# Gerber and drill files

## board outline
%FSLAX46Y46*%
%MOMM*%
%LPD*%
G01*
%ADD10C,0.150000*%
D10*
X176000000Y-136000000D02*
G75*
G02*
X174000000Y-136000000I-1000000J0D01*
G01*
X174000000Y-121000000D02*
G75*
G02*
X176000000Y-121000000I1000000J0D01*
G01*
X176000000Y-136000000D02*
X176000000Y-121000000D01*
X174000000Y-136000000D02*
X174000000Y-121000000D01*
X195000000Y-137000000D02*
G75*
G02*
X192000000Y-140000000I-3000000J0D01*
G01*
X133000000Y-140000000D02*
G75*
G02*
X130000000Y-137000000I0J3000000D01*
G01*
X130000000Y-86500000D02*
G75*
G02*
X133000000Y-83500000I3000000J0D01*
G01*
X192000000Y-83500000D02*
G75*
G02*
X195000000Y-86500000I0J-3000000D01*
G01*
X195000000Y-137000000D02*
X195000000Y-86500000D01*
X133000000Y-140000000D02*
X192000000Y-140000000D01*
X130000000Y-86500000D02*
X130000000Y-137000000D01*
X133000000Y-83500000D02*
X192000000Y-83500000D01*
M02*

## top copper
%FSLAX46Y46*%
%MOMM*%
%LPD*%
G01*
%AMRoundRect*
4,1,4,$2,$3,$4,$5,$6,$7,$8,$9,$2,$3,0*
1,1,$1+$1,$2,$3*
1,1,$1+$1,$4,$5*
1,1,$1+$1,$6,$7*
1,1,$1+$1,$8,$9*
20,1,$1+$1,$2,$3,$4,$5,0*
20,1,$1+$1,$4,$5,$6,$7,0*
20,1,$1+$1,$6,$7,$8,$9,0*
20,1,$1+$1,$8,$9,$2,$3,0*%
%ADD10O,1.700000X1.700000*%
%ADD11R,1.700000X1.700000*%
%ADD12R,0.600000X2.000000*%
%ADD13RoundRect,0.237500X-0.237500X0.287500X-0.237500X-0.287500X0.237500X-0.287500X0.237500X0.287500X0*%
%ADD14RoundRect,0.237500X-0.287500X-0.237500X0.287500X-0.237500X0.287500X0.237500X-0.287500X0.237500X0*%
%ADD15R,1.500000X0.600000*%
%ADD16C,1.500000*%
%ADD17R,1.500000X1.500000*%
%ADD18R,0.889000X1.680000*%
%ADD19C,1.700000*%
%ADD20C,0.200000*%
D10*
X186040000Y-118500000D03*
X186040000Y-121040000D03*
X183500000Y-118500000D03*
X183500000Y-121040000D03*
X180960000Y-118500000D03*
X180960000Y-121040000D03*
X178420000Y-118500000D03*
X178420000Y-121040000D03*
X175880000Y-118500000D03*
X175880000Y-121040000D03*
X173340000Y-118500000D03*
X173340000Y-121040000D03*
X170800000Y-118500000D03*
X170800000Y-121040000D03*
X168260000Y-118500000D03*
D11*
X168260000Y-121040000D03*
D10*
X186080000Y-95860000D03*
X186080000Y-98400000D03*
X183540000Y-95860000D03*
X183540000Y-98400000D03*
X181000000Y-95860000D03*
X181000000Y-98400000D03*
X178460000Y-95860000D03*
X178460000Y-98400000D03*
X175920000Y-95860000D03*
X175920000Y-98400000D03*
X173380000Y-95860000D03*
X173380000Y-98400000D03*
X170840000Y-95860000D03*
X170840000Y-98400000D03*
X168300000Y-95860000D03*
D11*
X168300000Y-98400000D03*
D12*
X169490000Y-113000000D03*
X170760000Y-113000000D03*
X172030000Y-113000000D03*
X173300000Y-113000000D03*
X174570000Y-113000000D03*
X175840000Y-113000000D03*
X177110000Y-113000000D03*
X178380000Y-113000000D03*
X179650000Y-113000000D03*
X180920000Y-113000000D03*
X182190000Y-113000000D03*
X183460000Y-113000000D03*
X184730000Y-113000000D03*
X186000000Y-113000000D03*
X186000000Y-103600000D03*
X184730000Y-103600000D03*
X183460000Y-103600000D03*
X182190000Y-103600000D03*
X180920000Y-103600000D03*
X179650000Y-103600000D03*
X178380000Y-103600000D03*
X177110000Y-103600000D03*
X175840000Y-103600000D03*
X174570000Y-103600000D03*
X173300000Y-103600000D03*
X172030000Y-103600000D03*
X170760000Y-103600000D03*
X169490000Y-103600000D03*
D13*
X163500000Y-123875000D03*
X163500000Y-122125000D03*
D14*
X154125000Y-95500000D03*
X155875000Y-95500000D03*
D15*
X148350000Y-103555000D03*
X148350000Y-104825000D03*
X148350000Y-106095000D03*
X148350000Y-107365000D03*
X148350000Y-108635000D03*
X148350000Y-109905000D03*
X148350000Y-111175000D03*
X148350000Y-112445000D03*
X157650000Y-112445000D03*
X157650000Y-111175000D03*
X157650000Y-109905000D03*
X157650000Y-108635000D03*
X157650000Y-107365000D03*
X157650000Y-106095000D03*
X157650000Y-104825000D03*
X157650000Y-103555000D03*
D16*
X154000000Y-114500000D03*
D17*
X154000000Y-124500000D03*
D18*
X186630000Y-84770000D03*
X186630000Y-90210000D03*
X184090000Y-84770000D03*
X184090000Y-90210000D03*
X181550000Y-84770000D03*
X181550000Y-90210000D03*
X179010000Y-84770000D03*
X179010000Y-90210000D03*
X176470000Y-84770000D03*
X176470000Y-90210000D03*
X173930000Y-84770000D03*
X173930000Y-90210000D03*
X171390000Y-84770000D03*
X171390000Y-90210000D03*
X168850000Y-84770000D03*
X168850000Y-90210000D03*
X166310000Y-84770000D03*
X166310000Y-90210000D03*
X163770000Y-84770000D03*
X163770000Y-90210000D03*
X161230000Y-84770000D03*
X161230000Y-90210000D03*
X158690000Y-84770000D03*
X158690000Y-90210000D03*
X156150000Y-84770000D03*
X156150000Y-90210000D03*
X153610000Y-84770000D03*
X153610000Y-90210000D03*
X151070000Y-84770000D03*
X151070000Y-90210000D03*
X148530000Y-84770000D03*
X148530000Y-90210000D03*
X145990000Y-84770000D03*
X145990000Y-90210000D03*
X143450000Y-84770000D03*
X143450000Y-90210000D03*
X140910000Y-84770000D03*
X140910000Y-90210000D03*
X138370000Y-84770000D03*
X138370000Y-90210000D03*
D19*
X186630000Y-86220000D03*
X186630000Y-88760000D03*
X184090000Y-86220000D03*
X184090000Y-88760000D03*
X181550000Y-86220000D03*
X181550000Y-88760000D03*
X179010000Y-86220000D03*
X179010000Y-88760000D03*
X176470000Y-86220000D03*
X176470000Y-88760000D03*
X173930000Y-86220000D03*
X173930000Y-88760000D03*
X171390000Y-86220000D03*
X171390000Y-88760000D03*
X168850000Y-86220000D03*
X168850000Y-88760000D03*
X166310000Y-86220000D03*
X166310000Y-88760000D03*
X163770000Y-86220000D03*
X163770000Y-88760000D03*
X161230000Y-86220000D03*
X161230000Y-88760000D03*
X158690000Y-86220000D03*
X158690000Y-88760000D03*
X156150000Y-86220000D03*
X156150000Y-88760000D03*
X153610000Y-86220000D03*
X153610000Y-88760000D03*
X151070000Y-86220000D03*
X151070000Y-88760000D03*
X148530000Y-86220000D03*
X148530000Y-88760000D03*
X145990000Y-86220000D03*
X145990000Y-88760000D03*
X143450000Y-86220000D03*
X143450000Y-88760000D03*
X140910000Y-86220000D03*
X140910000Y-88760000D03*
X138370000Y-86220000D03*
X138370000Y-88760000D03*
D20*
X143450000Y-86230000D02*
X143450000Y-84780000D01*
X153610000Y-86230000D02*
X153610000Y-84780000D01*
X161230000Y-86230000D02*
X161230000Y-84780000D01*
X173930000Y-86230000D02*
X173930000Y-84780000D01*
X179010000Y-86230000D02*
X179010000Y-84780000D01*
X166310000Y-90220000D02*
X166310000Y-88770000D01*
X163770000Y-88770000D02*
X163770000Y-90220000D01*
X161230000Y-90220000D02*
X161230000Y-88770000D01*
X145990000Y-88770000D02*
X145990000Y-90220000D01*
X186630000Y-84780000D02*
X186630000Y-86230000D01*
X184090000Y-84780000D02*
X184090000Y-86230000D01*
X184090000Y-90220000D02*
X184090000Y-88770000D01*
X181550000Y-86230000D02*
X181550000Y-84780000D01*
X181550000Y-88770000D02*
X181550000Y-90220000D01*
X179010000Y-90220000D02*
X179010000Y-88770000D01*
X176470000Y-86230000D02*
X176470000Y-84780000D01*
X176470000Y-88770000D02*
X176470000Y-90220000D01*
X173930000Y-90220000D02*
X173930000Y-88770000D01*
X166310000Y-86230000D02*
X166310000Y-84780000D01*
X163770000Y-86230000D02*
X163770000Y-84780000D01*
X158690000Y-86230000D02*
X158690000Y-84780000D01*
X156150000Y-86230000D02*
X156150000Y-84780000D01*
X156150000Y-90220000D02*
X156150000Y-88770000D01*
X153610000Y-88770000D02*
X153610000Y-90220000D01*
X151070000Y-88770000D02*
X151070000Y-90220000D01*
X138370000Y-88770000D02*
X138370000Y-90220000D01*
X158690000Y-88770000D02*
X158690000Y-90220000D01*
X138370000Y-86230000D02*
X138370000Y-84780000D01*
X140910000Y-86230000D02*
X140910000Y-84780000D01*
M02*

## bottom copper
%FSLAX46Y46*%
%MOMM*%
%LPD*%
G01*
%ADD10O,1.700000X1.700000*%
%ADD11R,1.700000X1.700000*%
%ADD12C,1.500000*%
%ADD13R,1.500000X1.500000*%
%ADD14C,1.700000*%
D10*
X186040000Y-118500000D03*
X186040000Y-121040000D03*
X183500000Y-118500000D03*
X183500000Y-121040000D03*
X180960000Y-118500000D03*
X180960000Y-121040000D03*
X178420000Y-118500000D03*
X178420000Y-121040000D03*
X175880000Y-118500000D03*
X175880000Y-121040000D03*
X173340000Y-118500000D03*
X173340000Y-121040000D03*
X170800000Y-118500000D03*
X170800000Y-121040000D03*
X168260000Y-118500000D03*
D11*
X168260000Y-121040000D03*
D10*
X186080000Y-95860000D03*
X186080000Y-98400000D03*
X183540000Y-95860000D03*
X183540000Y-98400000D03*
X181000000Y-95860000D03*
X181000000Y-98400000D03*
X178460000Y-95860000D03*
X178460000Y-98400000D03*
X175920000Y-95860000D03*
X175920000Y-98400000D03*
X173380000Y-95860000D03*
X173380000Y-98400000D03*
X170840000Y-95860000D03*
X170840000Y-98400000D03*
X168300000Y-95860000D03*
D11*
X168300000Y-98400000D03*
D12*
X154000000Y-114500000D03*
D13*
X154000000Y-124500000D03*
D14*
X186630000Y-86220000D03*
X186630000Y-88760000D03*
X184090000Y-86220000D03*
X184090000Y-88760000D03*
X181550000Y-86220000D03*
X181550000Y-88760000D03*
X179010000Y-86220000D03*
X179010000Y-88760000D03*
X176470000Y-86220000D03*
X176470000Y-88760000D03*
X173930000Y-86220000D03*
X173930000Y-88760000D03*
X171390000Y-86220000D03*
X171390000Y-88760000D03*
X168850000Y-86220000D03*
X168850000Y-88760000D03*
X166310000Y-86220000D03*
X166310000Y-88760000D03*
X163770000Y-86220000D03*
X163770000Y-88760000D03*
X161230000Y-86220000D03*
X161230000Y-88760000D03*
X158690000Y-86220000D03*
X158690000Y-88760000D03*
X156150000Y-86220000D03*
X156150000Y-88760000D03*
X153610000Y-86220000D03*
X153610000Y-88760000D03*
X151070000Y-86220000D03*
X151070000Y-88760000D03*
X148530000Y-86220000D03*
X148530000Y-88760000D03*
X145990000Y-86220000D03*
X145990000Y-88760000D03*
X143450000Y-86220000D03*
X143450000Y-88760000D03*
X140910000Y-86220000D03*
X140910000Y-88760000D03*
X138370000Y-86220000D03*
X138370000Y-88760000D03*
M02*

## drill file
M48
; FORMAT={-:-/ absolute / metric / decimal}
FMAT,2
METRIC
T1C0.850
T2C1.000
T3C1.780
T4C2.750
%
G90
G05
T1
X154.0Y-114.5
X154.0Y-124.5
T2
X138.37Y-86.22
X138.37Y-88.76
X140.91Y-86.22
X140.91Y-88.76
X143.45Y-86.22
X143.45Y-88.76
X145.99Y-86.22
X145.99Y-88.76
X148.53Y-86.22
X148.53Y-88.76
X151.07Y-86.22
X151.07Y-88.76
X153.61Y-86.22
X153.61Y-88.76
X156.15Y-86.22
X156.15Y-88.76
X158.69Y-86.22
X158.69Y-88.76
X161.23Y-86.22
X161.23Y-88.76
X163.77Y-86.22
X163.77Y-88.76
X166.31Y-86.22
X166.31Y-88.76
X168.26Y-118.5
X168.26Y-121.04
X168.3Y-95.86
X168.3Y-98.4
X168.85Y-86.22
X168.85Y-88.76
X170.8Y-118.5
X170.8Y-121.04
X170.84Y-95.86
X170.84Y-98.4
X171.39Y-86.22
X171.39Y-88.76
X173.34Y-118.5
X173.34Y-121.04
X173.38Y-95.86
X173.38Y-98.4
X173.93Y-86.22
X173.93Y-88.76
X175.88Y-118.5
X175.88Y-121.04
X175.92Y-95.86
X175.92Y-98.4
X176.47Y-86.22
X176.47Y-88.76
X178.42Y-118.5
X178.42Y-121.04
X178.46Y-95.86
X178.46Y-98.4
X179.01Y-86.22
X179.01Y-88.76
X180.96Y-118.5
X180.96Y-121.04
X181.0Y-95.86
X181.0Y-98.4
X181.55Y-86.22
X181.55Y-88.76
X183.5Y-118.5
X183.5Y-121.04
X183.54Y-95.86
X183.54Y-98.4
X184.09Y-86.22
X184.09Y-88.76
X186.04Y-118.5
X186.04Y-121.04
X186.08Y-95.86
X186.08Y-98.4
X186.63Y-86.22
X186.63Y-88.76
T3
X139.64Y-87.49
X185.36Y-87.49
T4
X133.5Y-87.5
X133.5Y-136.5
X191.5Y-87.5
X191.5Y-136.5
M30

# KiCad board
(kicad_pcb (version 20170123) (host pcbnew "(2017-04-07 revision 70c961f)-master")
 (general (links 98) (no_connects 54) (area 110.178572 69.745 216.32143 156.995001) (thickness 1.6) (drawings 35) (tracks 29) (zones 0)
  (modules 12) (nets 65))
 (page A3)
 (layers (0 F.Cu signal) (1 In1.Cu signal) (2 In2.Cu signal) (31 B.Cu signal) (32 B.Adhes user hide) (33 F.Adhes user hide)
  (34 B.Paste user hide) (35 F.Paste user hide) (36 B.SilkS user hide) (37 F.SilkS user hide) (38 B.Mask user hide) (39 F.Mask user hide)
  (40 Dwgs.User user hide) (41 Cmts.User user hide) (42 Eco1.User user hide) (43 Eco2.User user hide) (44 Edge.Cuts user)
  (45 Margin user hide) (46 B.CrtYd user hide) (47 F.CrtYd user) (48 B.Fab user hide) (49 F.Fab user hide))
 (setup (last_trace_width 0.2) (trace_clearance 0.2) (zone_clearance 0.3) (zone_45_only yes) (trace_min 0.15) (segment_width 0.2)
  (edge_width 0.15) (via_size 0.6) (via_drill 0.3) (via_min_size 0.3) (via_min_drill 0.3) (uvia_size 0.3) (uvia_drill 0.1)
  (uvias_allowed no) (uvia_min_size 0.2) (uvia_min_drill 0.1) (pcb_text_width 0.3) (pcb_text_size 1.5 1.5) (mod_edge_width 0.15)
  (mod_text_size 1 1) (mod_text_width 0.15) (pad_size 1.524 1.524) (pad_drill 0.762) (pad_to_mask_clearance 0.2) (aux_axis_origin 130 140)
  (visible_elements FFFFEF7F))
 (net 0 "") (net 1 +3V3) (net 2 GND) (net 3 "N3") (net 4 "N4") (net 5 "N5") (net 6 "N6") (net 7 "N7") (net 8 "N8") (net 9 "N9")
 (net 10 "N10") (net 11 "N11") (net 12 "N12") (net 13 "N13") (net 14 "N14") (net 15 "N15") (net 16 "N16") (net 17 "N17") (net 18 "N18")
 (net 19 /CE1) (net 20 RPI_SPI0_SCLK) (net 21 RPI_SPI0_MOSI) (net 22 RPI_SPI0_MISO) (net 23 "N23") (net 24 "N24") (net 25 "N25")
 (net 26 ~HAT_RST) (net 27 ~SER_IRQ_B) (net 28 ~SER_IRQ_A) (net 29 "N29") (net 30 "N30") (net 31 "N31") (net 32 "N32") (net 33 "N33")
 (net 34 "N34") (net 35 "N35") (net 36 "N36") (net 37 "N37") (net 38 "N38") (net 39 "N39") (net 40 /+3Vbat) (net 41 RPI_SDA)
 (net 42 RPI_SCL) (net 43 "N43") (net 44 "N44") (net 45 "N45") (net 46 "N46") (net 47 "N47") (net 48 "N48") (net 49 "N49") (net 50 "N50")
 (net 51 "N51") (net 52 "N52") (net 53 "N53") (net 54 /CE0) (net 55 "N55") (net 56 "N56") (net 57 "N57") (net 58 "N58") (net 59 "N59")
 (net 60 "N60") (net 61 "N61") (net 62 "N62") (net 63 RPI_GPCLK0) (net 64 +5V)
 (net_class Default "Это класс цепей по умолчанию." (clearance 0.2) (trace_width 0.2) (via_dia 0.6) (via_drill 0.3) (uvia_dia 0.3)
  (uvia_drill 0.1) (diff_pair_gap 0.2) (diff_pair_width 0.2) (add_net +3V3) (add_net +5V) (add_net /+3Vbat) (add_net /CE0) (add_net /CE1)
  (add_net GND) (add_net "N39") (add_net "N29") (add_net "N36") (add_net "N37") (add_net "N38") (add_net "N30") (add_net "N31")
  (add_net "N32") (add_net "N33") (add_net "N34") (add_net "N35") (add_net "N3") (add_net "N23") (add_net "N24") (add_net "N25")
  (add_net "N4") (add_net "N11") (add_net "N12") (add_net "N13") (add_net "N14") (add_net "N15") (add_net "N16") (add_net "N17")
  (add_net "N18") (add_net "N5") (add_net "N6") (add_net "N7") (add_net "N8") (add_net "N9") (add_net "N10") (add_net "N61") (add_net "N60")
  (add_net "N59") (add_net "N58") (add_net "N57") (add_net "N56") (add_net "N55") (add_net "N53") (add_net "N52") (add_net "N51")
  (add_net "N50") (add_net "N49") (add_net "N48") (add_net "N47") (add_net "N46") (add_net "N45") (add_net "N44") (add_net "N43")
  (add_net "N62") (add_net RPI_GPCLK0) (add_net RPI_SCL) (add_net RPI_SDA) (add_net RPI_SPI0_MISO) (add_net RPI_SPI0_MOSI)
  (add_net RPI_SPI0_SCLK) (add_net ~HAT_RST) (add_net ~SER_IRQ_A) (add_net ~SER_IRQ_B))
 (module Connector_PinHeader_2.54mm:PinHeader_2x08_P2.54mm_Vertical (layer F.Cu) (at 168.26 121.04 90)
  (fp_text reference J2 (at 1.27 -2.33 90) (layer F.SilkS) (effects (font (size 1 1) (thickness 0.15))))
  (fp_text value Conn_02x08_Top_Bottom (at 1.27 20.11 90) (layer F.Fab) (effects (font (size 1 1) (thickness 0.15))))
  (pad 16 thru_hole oval (at 2.54 17.78 90) (size 1.7 1.7) (drill 1) (layers *.Cu *.Mask) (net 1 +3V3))
  (pad 15 thru_hole oval (at 0 17.78 90) (size 1.7 1.7) (drill 1) (layers *.Cu *.Mask) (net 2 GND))
  (pad 14 thru_hole oval (at 2.54 15.24 90) (size 1.7 1.7) (drill 1) (layers *.Cu *.Mask) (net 1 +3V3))
  (pad 13 thru_hole oval (at 0 15.24 90) (size 1.7 1.7) (drill 1) (layers *.Cu *.Mask) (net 2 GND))
  (pad 12 thru_hole oval (at 2.54 12.7 90) (size 1.7 1.7) (drill 1) (layers *.Cu *.Mask) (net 1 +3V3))
  (pad 11 thru_hole oval (at 0 12.7 90) (size 1.7 1.7) (drill 1) (layers *.Cu *.Mask) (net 2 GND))
  (pad 10 thru_hole oval (at 2.54 10.16 90) (size 1.7 1.7) (drill 1) (layers *.Cu *.Mask) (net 1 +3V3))
  (pad 9 thru_hole oval (at 0 10.16 90) (size 1.7 1.7) (drill 1) (layers *.Cu *.Mask) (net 2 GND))
  (pad 8 thru_hole oval (at 2.54 7.62 90) (size 1.7 1.7) (drill 1) (layers *.Cu *.Mask) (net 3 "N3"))
  (pad 7 thru_hole oval (at 0 7.62 90) (size 1.7 1.7) (drill 1) (layers *.Cu *.Mask) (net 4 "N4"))
  (pad 6 thru_hole oval (at 2.54 5.08 90) (size 1.7 1.7) (drill 1) (layers *.Cu *.Mask) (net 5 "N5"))
  (pad 5 thru_hole oval (at 0 5.08 90) (size 1.7 1.7) (drill 1) (layers *.Cu *.Mask) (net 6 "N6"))
  (pad 4 thru_hole oval (at 2.54 2.54 90) (size 1.7 1.7) (drill 1) (layers *.Cu *.Mask) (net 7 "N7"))
  (pad 3 thru_hole oval (at 0 2.54 90) (size 1.7 1.7) (drill 1) (layers *.Cu *.Mask) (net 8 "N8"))
  (pad 2 thru_hole oval (at 2.54 0 90) (size 1.7 1.7) (drill 1) (layers *.Cu *.Mask) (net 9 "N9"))
  (pad 1 thru_hole rect (at 0 0 90) (size 1.7 1.7) (drill 1) (layers *.Cu *.Mask) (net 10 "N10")))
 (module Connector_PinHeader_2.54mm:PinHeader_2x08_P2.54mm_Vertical (layer F.Cu) (at 168.3 98.4 90)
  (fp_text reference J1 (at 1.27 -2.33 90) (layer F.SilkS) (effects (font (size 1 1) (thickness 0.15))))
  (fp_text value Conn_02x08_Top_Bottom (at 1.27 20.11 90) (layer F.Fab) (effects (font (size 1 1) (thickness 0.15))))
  (pad 16 thru_hole oval (at 2.54 17.78 90) (size 1.7 1.7) (drill 1) (layers *.Cu *.Mask) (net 1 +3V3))
  (pad 15 thru_hole oval (at 0 17.78 90) (size 1.7 1.7) (drill 1) (layers *.Cu *.Mask) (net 2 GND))
  (pad 14 thru_hole oval (at 2.54 15.24 90) (size 1.7 1.7) (drill 1) (layers *.Cu *.Mask) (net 1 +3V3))
  (pad 13 thru_hole oval (at 0 15.24 90) (size 1.7 1.7) (drill 1) (layers *.Cu *.Mask) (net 2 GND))
  (pad 12 thru_hole oval (at 2.54 12.7 90) (size 1.7 1.7) (drill 1) (layers *.Cu *.Mask) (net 1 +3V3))
  (pad 11 thru_hole oval (at 0 12.7 90) (size 1.7 1.7) (drill 1) (layers *.Cu *.Mask) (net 2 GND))
  (pad 10 thru_hole oval (at 2.54 10.16 90) (size 1.7 1.7) (drill 1) (layers *.Cu *.Mask) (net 1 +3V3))
  (pad 9 thru_hole oval (at 0 10.16 90) (size 1.7 1.7) (drill 1) (layers *.Cu *.Mask) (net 2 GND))
  (pad 8 thru_hole oval (at 2.54 7.62 90) (size 1.7 1.7) (drill 1) (layers *.Cu *.Mask) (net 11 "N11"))
  (pad 7 thru_hole oval (at 0 7.62 90) (size 1.7 1.7) (drill 1) (layers *.Cu *.Mask) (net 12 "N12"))
  (pad 6 thru_hole oval (at 2.54 5.08 90) (size 1.7 1.7) (drill 1) (layers *.Cu *.Mask) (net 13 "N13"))
  (pad 5 thru_hole oval (at 0 5.08 90) (size 1.7 1.7) (drill 1) (layers *.Cu *.Mask) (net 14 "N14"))
  (pad 4 thru_hole oval (at 2.54 2.54 90) (size 1.7 1.7) (drill 1) (layers *.Cu *.Mask) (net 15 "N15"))
  (pad 3 thru_hole oval (at 0 2.54 90) (size 1.7 1.7) (drill 1) (layers *.Cu *.Mask) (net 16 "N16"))
  (pad 2 thru_hole oval (at 2.54 0 90) (size 1.7 1.7) (drill 1) (layers *.Cu *.Mask) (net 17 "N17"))
  (pad 1 thru_hole rect (at 0 0 90) (size 1.7 1.7) (drill 1) (layers *.Cu *.Mask) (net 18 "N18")))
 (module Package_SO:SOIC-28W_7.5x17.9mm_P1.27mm (layer F.Cu) (at 177.745 108.3 90)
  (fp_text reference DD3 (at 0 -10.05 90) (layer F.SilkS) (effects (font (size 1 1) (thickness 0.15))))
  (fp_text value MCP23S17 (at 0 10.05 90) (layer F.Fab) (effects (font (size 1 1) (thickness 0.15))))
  (pad 1 smd rect (at -4.7 -8.255 90) (size 2 0.6) (layers F.Cu F.Paste F.Mask) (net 3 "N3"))
  (pad 2 smd rect (at -4.7 -6.985 90) (size 2 0.6) (layers F.Cu F.Paste F.Mask) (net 4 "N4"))
  (pad 3 smd rect (at -4.7 -5.715 90) (size 2 0.6) (layers F.Cu F.Paste F.Mask) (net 5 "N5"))
  (pad 4 smd rect (at -4.7 -4.445 90) (size 2 0.6) (layers F.Cu F.Paste F.Mask) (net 6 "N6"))
  (pad 5 smd rect (at -4.7 -3.175 90) (size 2 0.6) (layers F.Cu F.Paste F.Mask) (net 7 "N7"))
  (pad 6 smd rect (at -4.7 -1.905 90) (size 2 0.6) (layers F.Cu F.Paste F.Mask) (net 8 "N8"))
  (pad 7 smd rect (at -4.7 -0.635 90) (size 2 0.6) (layers F.Cu F.Paste F.Mask) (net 9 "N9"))
  (pad 8 smd rect (at -4.7 0.635 90) (size 2 0.6) (layers F.Cu F.Paste F.Mask) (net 10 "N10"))
  (pad 9 smd rect (at -4.7 1.905 90) (size 2 0.6) (layers F.Cu F.Paste F.Mask) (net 1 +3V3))
  (pad 10 smd rect (at -4.7 3.175 90) (size 2 0.6) (layers F.Cu F.Paste F.Mask) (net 2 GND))
  (pad 11 smd rect (at -4.7 4.445 90) (size 2 0.6) (layers F.Cu F.Paste F.Mask) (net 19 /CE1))
  (pad 12 smd rect (at -4.7 5.715 90) (size 2 0.6) (layers F.Cu F.Paste F.Mask) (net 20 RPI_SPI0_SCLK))
  (pad 13 smd rect (at -4.7 6.985 90) (size 2 0.6) (layers F.Cu F.Paste F.Mask) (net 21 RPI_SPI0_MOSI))
  (pad 14 smd rect (at -4.7 8.255 90) (size 2 0.6) (layers F.Cu F.Paste F.Mask) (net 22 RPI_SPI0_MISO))
  (pad 15 smd rect (at 4.7 8.255 90) (size 2 0.6) (layers F.Cu F.Paste F.Mask) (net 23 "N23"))
  (pad 16 smd rect (at 4.7 6.985 90) (size 2 0.6) (layers F.Cu F.Paste F.Mask) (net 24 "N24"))
  (pad 17 smd rect (at 4.7 5.715 90) (size 2 0.6) (layers F.Cu F.Paste F.Mask) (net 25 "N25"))
  (pad 18 smd rect (at 4.7 4.445 90) (size 2 0.6) (layers F.Cu F.Paste F.Mask) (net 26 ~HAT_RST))
  (pad 19 smd rect (at 4.7 3.175 90) (size 2 0.6) (layers F.Cu F.Paste F.Mask) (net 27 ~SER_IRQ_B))
  (pad 20 smd rect (at 4.7 1.905 90) (size 2 0.6) (layers F.Cu F.Paste F.Mask) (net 27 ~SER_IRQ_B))
  (pad 21 smd rect (at 4.7 0.635 90) (size 2 0.6) (layers F.Cu F.Paste F.Mask) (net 11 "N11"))
  (pad 22 smd rect (at 4.7 -0.635 90) (size 2 0.6) (layers F.Cu F.Paste F.Mask) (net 12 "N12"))
  (pad 23 smd rect (at 4.7 -1.905 90) (size 2 0.6) (layers F.Cu F.Paste F.Mask) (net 13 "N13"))
  (pad 24 smd rect (at 4.7 -3.175 90) (size 2 0.6) (layers F.Cu F.Paste F.Mask) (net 14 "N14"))
  (pad 25 smd rect (at 4.7 -4.445 90) (size 2 0.6) (layers F.Cu F.Paste F.Mask) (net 15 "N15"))
  (pad 26 smd rect (at 4.7 -5.715 90) (size 2 0.6) (layers F.Cu F.Paste F.Mask) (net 16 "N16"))
  (pad 27 smd rect (at 4.7 -6.985 90) (size 2 0.6) (layers F.Cu F.Paste F.Mask) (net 17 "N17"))
  (pad 28 smd rect (at 4.7 -8.255 90) (size 2 0.6) (layers F.Cu F.Paste F.Mask) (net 18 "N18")))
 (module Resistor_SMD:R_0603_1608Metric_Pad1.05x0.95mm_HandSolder (layer F.Cu) (at 163.5 123 270)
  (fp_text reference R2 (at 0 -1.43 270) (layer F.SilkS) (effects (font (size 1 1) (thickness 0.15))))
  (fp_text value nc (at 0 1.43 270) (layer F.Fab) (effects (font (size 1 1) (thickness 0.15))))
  (pad 2 smd roundrect (at 0.875 0 270) (size 1.05 0.95) (layers F.Cu F.Paste F.Mask) (roundrect_rratio 0.25) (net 1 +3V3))
  (pad 1 smd roundrect (at -0.875 0 270) (size 1.05 0.95) (layers F.Cu F.Paste F.Mask) (roundrect_rratio 0.25) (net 26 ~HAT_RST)))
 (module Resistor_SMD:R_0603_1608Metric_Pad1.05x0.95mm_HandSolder (layer F.Cu) (at 155 95.5)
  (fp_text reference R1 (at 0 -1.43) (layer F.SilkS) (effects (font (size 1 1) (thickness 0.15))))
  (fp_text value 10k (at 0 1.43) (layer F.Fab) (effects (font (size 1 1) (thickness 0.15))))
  (pad 1 smd roundrect (at -0.875 0) (size 1.05 0.95) (layers F.Cu F.Paste F.Mask) (roundrect_rratio 0.25) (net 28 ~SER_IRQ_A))
  (pad 2 smd roundrect (at 0.875 0) (size 1.05 0.95) (layers F.Cu F.Paste F.Mask) (roundrect_rratio 0.25) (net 1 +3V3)))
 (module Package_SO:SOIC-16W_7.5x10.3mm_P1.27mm (layer F.Cu) (at 153 108)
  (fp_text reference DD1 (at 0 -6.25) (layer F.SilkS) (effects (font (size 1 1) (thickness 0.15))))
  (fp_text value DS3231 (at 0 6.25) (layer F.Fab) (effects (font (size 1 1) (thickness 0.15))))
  (pad 1 smd rect (at -4.65 -4.445) (size 1.5 0.6) (layers F.Cu F.Paste F.Mask) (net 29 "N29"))
  (pad 2 smd rect (at -4.65 -3.175) (size 1.5 0.6) (layers F.Cu F.Paste F.Mask) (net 1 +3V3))
  (pad 3 smd rect (at -4.65 -1.905) (size 1.5 0.6) (layers F.Cu F.Paste F.Mask) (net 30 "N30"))
  (pad 4 smd rect (at -4.65 -0.635) (size 1.5 0.6) (layers F.Cu F.Paste F.Mask) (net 26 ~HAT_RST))
  (pad 5 smd rect (at -4.65 0.635) (size 1.5 0.6) (layers F.Cu F.Paste F.Mask) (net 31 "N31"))
  (pad 6 smd rect (at -4.65 1.905) (size 1.5 0.6) (layers F.Cu F.Paste F.Mask) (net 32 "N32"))
  (pad 7 smd rect (at -4.65 3.175) (size 1.5 0.6) (layers F.Cu F.Paste F.Mask) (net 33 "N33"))
  (pad 8 smd rect (at -4.65 4.445) (size 1.5 0.6) (layers F.Cu F.Paste F.Mask) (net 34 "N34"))
  (pad 9 smd rect (at 4.65 4.445) (size 1.5 0.6) (layers F.Cu F.Paste F.Mask) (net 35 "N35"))
  (pad 10 smd rect (at 4.65 3.175) (size 1.5 0.6) (layers F.Cu F.Paste F.Mask) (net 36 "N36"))
  (pad 11 smd rect (at 4.65 1.905) (size 1.5 0.6) (layers F.Cu F.Paste F.Mask) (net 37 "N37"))
  (pad 12 smd rect (at 4.65 0.635) (size 1.5 0.6) (layers F.Cu F.Paste F.Mask) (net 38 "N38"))
  (pad 13 smd rect (at 4.65 -0.635) (size 1.5 0.6) (layers F.Cu F.Paste F.Mask) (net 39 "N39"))
  (pad 14 smd rect (at 4.65 -1.905) (size 1.5 0.6) (layers F.Cu F.Paste F.Mask) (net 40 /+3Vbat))
  (pad 15 smd rect (at 4.65 -3.175) (size 1.5 0.6) (layers F.Cu F.Paste F.Mask) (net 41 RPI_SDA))
  (pad 16 smd rect (at 4.65 -4.445) (size 1.5 0.6) (layers F.Cu F.Paste F.Mask) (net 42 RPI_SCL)))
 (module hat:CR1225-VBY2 (layer F.Cu) (at 154 119.5 90)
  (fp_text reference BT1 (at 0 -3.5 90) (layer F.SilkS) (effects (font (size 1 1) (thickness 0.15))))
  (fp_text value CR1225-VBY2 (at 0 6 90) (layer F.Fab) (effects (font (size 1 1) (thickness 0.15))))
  (pad 2 thru_hole circle (at 5 0 90) (size 1.5 1.5) (drill 0.85) (layers *.Cu *.Mask) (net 39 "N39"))
  (pad 1 thru_hole rect (at -5 0 90) (size 1.5 1.5) (drill 0.85) (layers *.Cu *.Mask) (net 40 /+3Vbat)))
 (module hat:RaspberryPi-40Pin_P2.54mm (layer F.Cu) (at 162.5 87.49)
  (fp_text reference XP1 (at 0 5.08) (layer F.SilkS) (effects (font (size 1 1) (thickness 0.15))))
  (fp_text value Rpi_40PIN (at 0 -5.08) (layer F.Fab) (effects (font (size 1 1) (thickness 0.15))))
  (pad "" np_thru_hole circle (at 22.86 0) (size 1.78 1.78) (drill 1.78) (layers *.Cu *.Mask))
  (pad "" np_thru_hole circle (at -22.86 0) (size 1.78 1.78) (drill 1.78) (layers *.Cu *.Mask))
  (pad 40 smd rect (at 24.13 -2.72) (size 0.889 1.68) (layers F.Cu F.Paste F.Mask) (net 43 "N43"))
  (pad 39 smd rect (at 24.13 2.72) (size 0.889 1.68) (layers F.Cu F.Paste F.Mask) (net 2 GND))
  (pad 38 smd rect (at 21.59 -2.72) (size 0.889 1.68) (layers F.Cu F.Paste F.Mask) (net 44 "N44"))
  (pad 37 smd rect (at 21.59 2.72) (size 0.889 1.68) (layers F.Cu F.Paste F.Mask) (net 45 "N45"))
  (pad 36 smd rect (at 19.05 -2.72) (size 0.889 1.68) (layers F.Cu F.Paste F.Mask) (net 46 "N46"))
  (pad 35 smd rect (at 19.05 2.72) (size 0.889 1.68) (layers F.Cu F.Paste F.Mask) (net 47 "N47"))
  (pad 34 smd rect (at 16.51 -2.72) (size 0.889 1.68) (layers F.Cu F.Paste F.Mask) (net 2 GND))
  (pad 33 smd rect (at 16.51 2.72) (size 0.889 1.68) (layers F.Cu F.Paste F.Mask) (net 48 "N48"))
  (pad 32 smd rect (at 13.97 -2.72) (size 0.889 1.68) (layers F.Cu F.Paste F.Mask) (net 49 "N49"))
  (pad 31 smd rect (at 13.97 2.72) (size 0.889 1.68) (layers F.Cu F.Paste F.Mask) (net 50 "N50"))
  (pad 30 smd rect (at 11.43 -2.72) (size 0.889 1.68) (layers F.Cu F.Paste F.Mask) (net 2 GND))
  (pad 29 smd rect (at 11.43 2.72) (size 0.889 1.68) (layers F.Cu F.Paste F.Mask) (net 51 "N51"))
  (pad 28 smd rect (at 8.89 -2.72) (size 0.889 1.68) (layers F.Cu F.Paste F.Mask) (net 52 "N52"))
  (pad 27 smd rect (at 8.89 2.72) (size 0.889 1.68) (layers F.Cu F.Paste F.Mask) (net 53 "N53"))
  (pad 26 smd rect (at 6.35 -2.72) (size 0.889 1.68) (layers F.Cu F.Paste F.Mask) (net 19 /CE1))
  (pad 25 smd rect (at 6.35 2.72) (size 0.889 1.68) (layers F.Cu F.Paste F.Mask) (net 2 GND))
  (pad 24 smd rect (at 3.81 -2.72) (size 0.889 1.68) (layers F.Cu F.Paste F.Mask) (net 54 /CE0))
  (pad 23 smd rect (at 3.81 2.72) (size 0.889 1.68) (layers F.Cu F.Paste F.Mask) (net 20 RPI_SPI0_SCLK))
  (pad 22 smd rect (at 1.27 -2.72) (size 0.889 1.68) (layers F.Cu F.Paste F.Mask) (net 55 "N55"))
  (pad 21 smd rect (at 1.27 2.72) (size 0.889 1.68) (layers F.Cu F.Paste F.Mask) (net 22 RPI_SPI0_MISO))
  (pad 20 smd rect (at -1.27 -2.72) (size 0.889 1.68) (layers F.Cu F.Paste F.Mask) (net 2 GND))
  (pad 19 smd rect (at -1.27 2.72) (size 0.889 1.68) (layers F.Cu F.Paste F.Mask) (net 21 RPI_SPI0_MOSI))
  (pad 18 smd rect (at -3.81 -2.72) (size 0.889 1.68) (layers F.Cu F.Paste F.Mask) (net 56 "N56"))
  (pad 17 smd rect (at -3.81 2.72) (size 0.889 1.68) (layers F.Cu F.Paste F.Mask) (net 1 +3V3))
  (pad 16 smd rect (at -6.35 -2.72) (size 0.889 1.68) (layers F.Cu F.Paste F.Mask) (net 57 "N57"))
  (pad 15 smd rect (at -6.35 2.72) (size 0.889 1.68) (layers F.Cu F.Paste F.Mask) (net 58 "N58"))
  (pad 14 smd rect (at -8.89 -2.72) (size 0.889 1.68) (layers F.Cu F.Paste F.Mask) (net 2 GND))
  (pad 13 smd rect (at -8.89 2.72) (size 0.889 1.68) (layers F.Cu F.Paste F.Mask) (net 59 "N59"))
  (pad 12 smd rect (at -11.43 -2.72) (size 0.889 1.68) (layers F.Cu F.Paste F.Mask) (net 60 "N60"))
  (pad 11 smd rect (at -11.43 2.72) (size 0.889 1.68) (layers F.Cu F.Paste F.Mask) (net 28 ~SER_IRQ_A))
  (pad 10 smd rect (at -13.97 -2.72) (size 0.889 1.68) (layers F.Cu F.Paste F.Mask) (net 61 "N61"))
  (pad 9 smd rect (at -13.97 2.72) (size 0.889 1.68) (layers F.Cu F.Paste F.Mask) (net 2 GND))
  (pad 8 smd rect (at -16.51 -2.72) (size 0.889 1.68) (layers F.Cu F.Paste F.Mask) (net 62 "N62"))
  (pad 7 smd rect (at -16.51 2.72) (size 0.889 1.68) (layers F.Cu F.Paste F.Mask) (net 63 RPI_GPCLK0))
  (pad 6 smd rect (at -19.05 -2.72) (size 0.889 1.68) (layers F.Cu F.Paste F.Mask) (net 2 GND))
  (pad 5 smd rect (at -19.05 2.72) (size 0.889 1.68) (layers F.Cu F.Paste F.Mask) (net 42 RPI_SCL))
  (pad 4 smd rect (at -21.59 -2.72) (size 0.889 1.68) (layers F.Cu F.Paste F.Mask) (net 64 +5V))
  (pad 3 smd rect (at -21.59 2.72) (size 0.889 1.68) (layers F.Cu F.Paste F.Mask) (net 41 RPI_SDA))
  (pad 2 smd rect (at -24.13 -2.72) (size 0.889 1.68) (layers F.Cu F.Paste F.Mask) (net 64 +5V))
  (pad 1 smd rect (at -24.13 2.72) (size 0.889 1.68) (layers F.Cu F.Paste F.Mask) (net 1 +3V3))
  (pad 40 thru_hole circle (at 24.13 -1.27) (size 1.7 1.7) (drill 1) (layers *.Cu *.Mask) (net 43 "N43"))
  (pad 39 thru_hole circle (at 24.13 1.27) (size 1.7 1.7) (drill 1) (layers *.Cu *.Mask) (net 2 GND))
  (pad 38 thru_hole circle (at 21.59 -1.27) (size 1.7 1.7) (drill 1) (layers *.Cu *.Mask) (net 44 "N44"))
  (pad 37 thru_hole circle (at 21.59 1.27) (size 1.7 1.7) (drill 1) (layers *.Cu *.Mask) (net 45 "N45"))
  (pad 36 thru_hole circle (at 19.05 -1.27) (size 1.7 1.7) (drill 1) (layers *.Cu *.Mask) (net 46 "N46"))
  (pad 35 thru_hole circle (at 19.05 1.27) (size 1.7 1.7) (drill 1) (layers *.Cu *.Mask) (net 47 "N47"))
  (pad 34 thru_hole circle (at 16.51 -1.27) (size 1.7 1.7) (drill 1) (layers *.Cu *.Mask) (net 2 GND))
  (pad 33 thru_hole circle (at 16.51 1.27) (size 1.7 1.7) (drill 1) (layers *.Cu *.Mask) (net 48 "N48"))
  (pad 32 thru_hole circle (at 13.97 -1.27) (size 1.7 1.7) (drill 1) (layers *.Cu *.Mask) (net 49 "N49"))
  (pad 31 thru_hole circle (at 13.97 1.27) (size 1.7 1.7) (drill 1) (layers *.Cu *.Mask) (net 50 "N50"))
  (pad 30 thru_hole circle (at 11.43 -1.27) (size 1.7 1.7) (drill 1) (layers *.Cu *.Mask) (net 2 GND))
  (pad 29 thru_hole circle (at 11.43 1.27) (size 1.7 1.7) (drill 1) (layers *.Cu *.Mask) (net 51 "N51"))
  (pad 28 thru_hole circle (at 8.89 -1.27) (size 1.7 1.7) (drill 1) (layers *.Cu *.Mask) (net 52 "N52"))
  (pad 27 thru_hole circle (at 8.89 1.27) (size 1.7 1.7) (drill 1) (layers *.Cu *.Mask) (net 53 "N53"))
  (pad 26 thru_hole circle (at 6.35 -1.27) (size 1.7 1.7) (drill 1) (layers *.Cu *.Mask) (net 19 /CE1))
  (pad 25 thru_hole circle (at 6.35 1.27) (size 1.7 1.7) (drill 1) (layers *.Cu *.Mask) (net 2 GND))
  (pad 24 thru_hole circle (at 3.81 -1.27) (size 1.7 1.7) (drill 1) (layers *.Cu *.Mask) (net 54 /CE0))
  (pad 23 thru_hole circle (at 3.81 1.27) (size 1.7 1.7) (drill 1) (layers *.Cu *.Mask) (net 20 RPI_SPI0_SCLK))
  (pad 22 thru_hole circle (at 1.27 -1.27) (size 1.7 1.7) (drill 1) (layers *.Cu *.Mask) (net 55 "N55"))
  (pad 21 thru_hole circle (at 1.27 1.27) (size 1.7 1.7) (drill 1) (layers *.Cu *.Mask) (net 22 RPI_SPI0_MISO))
  (pad 20 thru_hole circle (at -1.27 -1.27) (size 1.7 1.7) (drill 1) (layers *.Cu *.Mask) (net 2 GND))
  (pad 19 thru_hole circle (at -1.27 1.27) (size 1.7 1.7) (drill 1) (layers *.Cu *.Mask) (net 21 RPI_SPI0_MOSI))
  (pad 18 thru_hole circle (at -3.81 -1.27) (size 1.7 1.7) (drill 1) (layers *.Cu *.Mask) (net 56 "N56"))
  (pad 17 thru_hole circle (at -3.81 1.27) (size 1.7 1.7) (drill 1) (layers *.Cu *.Mask) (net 1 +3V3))
  (pad 16 thru_hole circle (at -6.35 -1.27) (size 1.7 1.7) (drill 1) (layers *.Cu *.Mask) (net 57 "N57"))
  (pad 15 thru_hole circle (at -6.35 1.27) (size 1.7 1.7) (drill 1) (layers *.Cu *.Mask) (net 58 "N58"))
  (pad 14 thru_hole circle (at -8.89 -1.27) (size 1.7 1.7) (drill 1) (layers *.Cu *.Mask) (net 2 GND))
  (pad 13 thru_hole circle (at -8.89 1.27) (size 1.7 1.7) (drill 1) (layers *.Cu *.Mask) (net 59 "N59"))
  (pad 12 thru_hole circle (at -11.43 -1.27) (size 1.7 1.7) (drill 1) (layers *.Cu *.Mask) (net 60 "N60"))
  (pad 11 thru_hole circle (at -11.43 1.27) (size 1.7 1.7) (drill 1) (layers *.Cu *.Mask) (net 28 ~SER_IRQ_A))
  (pad 10 thru_hole circle (at -13.97 -1.27) (size 1.7 1.7) (drill 1) (layers *.Cu *.Mask) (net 61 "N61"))
  (pad 9 thru_hole circle (at -13.97 1.27) (size 1.7 1.7) (drill 1) (layers *.Cu *.Mask) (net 2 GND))
  (pad 8 thru_hole circle (at -16.51 -1.27) (size 1.7 1.7) (drill 1) (layers *.Cu *.Mask) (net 62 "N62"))
  (pad 7 thru_hole circle (at -16.51 1.27) (size 1.7 1.7) (drill 1) (layers *.Cu *.Mask) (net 63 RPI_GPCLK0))
  (pad 6 thru_hole circle (at -19.05 -1.27) (size 1.7 1.7) (drill 1) (layers *.Cu *.Mask) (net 2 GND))
  (pad 5 thru_hole circle (at -19.05 1.27) (size 1.7 1.7) (drill 1) (layers *.Cu *.Mask) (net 42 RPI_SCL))
  (pad 4 thru_hole circle (at -21.59 -1.27) (size 1.7 1.7) (drill 1) (layers *.Cu *.Mask) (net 64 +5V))
  (pad 3 thru_hole circle (at -21.59 1.27) (size 1.7 1.7) (drill 1) (layers *.Cu *.Mask) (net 41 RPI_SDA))
  (pad 2 thru_hole circle (at -24.13 -1.27) (size 1.7 1.7) (drill 1) (layers *.Cu *.Mask) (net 64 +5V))
  (pad 1 thru_hole circle (at -24.13 1.27) (size 1.7 1.7) (drill 1) (layers *.Cu *.Mask) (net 1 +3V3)))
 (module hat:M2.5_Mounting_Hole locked (layer F.Cu) (at 133.5 87.5)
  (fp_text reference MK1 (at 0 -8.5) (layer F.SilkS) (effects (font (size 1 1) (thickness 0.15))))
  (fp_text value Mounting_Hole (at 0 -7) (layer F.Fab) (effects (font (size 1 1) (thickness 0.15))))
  (pad "" np_thru_hole circle (at 0 0) (size 2.75 2.75) (drill 2.75) (layers *.Cu *.Mask) (solder_mask_margin 1.8) (clearance 1.8)))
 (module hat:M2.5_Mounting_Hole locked (layer F.Cu) (at 191.5 87.5)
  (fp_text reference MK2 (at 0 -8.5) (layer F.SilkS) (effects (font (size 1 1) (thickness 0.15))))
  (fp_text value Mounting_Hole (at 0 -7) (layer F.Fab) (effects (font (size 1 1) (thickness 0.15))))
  (pad "" np_thru_hole circle (at 0 0) (size 2.75 2.75) (drill 2.75) (layers *.Cu *.Mask) (solder_mask_margin 1.8) (clearance 1.8)))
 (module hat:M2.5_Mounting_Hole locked (layer F.Cu) (at 133.5 136.5)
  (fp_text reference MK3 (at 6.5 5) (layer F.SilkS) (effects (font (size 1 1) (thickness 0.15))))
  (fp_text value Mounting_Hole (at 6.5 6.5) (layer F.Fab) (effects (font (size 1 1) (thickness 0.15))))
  (pad "" np_thru_hole circle (at 0 0) (size 2.75 2.75) (drill 2.75) (layers *.Cu *.Mask) (solder_mask_margin 1.8) (clearance 1.8)))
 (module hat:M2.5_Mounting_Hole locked (layer F.Cu) (at 191.5 136.5)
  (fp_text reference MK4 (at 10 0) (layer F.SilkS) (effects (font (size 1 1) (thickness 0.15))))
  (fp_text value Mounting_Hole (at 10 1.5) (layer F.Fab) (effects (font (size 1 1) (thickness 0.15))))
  (pad "" np_thru_hole circle (at 0 0) (size 2.75 2.75) (drill 2.75) (layers *.Cu *.Mask) (solder_mask_margin 1.8) (clearance 1.8)))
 (gr_arc (start 175 136) (end 174 136) (angle -180) (layer Edge.Cuts) (width 0.15))
 (gr_arc (start 175 121) (end 176 121) (angle -180) (layer Edge.Cuts) (width 0.15))
 (gr_line (start 176 136) (end 176 121) (layer Edge.Cuts) (width 0.15))
 (gr_line (start 174 136) (end 174 121) (layer Edge.Cuts) (width 0.15))
 (gr_arc (start 192 137) (end 195 137) (angle 90) (layer Edge.Cuts) (width 0.15))
 (gr_arc (start 133 137) (end 133 140) (angle 90) (layer Edge.Cuts) (width 0.15))
 (gr_arc (start 133 86.5) (end 130 86.5) (angle 90) (layer Edge.Cuts) (width 0.15))
 (gr_arc (start 192 86.5) (end 192 83.5) (angle 90) (layer Edge.Cuts) (width 0.15))
 (gr_line (start 195 137) (end 195 86.5) (layer Edge.Cuts) (width 0.15))
 (gr_line (start 133 140) (end 192 140) (layer Edge.Cuts) (width 0.15))
 (gr_line (start 130 86.5) (end 130 137) (layer Edge.Cuts) (width 0.15))
 (gr_line (start 133 83.5) (end 192 83.5) (layer Edge.Cuts) (width 0.15))
 (segment (start 143.45 86.23) (end 143.45 84.78) (width 0.2) (layer F.Cu) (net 2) (status 30))
 (segment (start 153.61 86.23) (end 153.61 84.78) (width 0.2) (layer F.Cu) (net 2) (status 30))
 (segment (start 161.23 86.23) (end 161.23 84.78) (width 0.2) (layer F.Cu) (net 2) (status 30))
 (segment (start 173.93 86.23) (end 173.93 84.78) (width 0.2) (layer F.Cu) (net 2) (status 30))
 (segment (start 179.01 86.23) (end 179.01 84.78) (width 0.2) (layer F.Cu) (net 2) (status 30))
 (segment (start 166.31 90.22) (end 166.31 88.77) (width 0.2) (layer F.Cu) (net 20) (status 30))
 (segment (start 163.77 88.77) (end 163.77 90.22) (width 0.2) (layer F.Cu) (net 22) (status 30))
 (segment (start 161.23 90.22) (end 161.23 88.77) (width 0.2) (layer F.Cu) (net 21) (status 30))
 (segment (start 145.99 88.77) (end 145.99 90.22) (width 0.2) (layer F.Cu) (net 63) (status 30))
 (segment (start 186.63 84.78) (end 186.63 86.23) (width 0.2) (layer F.Cu) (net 43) (status 30))
 (segment (start 184.09 84.78) (end 184.09 86.23) (width 0.2) (layer F.Cu) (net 44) (status 30))
 (segment (start 184.09 90.22) (end 184.09 88.77) (width 0.2) (layer F.Cu) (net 45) (status 30))
 (segment (start 181.55 86.23) (end 181.55 84.78) (width 0.2) (layer F.Cu) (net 46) (status 30))
 (segment (start 181.55 88.77) (end 181.55 90.22) (width 0.2) (layer F.Cu) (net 47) (status 30))
 (segment (start 179.01 90.22) (end 179.01 88.77) (width 0.2) (layer F.Cu) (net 48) (status 30))
 (segment (start 176.47 86.23) (end 176.47 84.78) (width 0.2) (layer F.Cu) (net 49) (status 30))
 (segment (start 176.47 88.77) (end 176.47 90.22) (width 0.2) (layer F.Cu) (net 50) (status 30))
 (segment (start 173.93 90.22) (end 173.93 88.77) (width 0.2) (layer F.Cu) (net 51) (status 30))
 (segment (start 166.31 86.23) (end 166.31 84.78) (width 0.2) (layer F.Cu) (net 54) (status 30))
 (segment (start 163.77 86.23) (end 163.77 84.78) (width 0.2) (layer F.Cu) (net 55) (status 30))
 (segment (start 158.69 86.23) (end 158.69 84.78) (width 0.2) (layer F.Cu) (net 56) (status 30))
 (segment (start 156.15 86.23) (end 156.15 84.78) (width 0.2) (layer F.Cu) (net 57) (status 30))
 (segment (start 156.15 90.22) (end 156.15 88.77) (width 0.2) (layer F.Cu) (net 58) (status 30))
 (segment (start 153.61 88.77) (end 153.61 90.22) (width 0.2) (layer F.Cu) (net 59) (status 30))
 (segment (start 151.07 88.77) (end 151.07 90.22) (width 0.2) (layer F.Cu) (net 28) (status 30))
 (segment (start 138.37 88.77) (end 138.37 90.22) (width 0.2) (layer F.Cu) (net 1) (status 30))
 (segment (start 158.69 88.77) (end 158.69 90.22) (width 0.2) (layer F.Cu) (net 1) (status 30))
 (segment (start 138.37 86.23) (end 138.37 84.78) (width 0.2) (layer F.Cu) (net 64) (status 30))
 (segment (start 140.91 86.23) (end 140.91 84.78) (width 0.2) (layer F.Cu) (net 64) (status 30)))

